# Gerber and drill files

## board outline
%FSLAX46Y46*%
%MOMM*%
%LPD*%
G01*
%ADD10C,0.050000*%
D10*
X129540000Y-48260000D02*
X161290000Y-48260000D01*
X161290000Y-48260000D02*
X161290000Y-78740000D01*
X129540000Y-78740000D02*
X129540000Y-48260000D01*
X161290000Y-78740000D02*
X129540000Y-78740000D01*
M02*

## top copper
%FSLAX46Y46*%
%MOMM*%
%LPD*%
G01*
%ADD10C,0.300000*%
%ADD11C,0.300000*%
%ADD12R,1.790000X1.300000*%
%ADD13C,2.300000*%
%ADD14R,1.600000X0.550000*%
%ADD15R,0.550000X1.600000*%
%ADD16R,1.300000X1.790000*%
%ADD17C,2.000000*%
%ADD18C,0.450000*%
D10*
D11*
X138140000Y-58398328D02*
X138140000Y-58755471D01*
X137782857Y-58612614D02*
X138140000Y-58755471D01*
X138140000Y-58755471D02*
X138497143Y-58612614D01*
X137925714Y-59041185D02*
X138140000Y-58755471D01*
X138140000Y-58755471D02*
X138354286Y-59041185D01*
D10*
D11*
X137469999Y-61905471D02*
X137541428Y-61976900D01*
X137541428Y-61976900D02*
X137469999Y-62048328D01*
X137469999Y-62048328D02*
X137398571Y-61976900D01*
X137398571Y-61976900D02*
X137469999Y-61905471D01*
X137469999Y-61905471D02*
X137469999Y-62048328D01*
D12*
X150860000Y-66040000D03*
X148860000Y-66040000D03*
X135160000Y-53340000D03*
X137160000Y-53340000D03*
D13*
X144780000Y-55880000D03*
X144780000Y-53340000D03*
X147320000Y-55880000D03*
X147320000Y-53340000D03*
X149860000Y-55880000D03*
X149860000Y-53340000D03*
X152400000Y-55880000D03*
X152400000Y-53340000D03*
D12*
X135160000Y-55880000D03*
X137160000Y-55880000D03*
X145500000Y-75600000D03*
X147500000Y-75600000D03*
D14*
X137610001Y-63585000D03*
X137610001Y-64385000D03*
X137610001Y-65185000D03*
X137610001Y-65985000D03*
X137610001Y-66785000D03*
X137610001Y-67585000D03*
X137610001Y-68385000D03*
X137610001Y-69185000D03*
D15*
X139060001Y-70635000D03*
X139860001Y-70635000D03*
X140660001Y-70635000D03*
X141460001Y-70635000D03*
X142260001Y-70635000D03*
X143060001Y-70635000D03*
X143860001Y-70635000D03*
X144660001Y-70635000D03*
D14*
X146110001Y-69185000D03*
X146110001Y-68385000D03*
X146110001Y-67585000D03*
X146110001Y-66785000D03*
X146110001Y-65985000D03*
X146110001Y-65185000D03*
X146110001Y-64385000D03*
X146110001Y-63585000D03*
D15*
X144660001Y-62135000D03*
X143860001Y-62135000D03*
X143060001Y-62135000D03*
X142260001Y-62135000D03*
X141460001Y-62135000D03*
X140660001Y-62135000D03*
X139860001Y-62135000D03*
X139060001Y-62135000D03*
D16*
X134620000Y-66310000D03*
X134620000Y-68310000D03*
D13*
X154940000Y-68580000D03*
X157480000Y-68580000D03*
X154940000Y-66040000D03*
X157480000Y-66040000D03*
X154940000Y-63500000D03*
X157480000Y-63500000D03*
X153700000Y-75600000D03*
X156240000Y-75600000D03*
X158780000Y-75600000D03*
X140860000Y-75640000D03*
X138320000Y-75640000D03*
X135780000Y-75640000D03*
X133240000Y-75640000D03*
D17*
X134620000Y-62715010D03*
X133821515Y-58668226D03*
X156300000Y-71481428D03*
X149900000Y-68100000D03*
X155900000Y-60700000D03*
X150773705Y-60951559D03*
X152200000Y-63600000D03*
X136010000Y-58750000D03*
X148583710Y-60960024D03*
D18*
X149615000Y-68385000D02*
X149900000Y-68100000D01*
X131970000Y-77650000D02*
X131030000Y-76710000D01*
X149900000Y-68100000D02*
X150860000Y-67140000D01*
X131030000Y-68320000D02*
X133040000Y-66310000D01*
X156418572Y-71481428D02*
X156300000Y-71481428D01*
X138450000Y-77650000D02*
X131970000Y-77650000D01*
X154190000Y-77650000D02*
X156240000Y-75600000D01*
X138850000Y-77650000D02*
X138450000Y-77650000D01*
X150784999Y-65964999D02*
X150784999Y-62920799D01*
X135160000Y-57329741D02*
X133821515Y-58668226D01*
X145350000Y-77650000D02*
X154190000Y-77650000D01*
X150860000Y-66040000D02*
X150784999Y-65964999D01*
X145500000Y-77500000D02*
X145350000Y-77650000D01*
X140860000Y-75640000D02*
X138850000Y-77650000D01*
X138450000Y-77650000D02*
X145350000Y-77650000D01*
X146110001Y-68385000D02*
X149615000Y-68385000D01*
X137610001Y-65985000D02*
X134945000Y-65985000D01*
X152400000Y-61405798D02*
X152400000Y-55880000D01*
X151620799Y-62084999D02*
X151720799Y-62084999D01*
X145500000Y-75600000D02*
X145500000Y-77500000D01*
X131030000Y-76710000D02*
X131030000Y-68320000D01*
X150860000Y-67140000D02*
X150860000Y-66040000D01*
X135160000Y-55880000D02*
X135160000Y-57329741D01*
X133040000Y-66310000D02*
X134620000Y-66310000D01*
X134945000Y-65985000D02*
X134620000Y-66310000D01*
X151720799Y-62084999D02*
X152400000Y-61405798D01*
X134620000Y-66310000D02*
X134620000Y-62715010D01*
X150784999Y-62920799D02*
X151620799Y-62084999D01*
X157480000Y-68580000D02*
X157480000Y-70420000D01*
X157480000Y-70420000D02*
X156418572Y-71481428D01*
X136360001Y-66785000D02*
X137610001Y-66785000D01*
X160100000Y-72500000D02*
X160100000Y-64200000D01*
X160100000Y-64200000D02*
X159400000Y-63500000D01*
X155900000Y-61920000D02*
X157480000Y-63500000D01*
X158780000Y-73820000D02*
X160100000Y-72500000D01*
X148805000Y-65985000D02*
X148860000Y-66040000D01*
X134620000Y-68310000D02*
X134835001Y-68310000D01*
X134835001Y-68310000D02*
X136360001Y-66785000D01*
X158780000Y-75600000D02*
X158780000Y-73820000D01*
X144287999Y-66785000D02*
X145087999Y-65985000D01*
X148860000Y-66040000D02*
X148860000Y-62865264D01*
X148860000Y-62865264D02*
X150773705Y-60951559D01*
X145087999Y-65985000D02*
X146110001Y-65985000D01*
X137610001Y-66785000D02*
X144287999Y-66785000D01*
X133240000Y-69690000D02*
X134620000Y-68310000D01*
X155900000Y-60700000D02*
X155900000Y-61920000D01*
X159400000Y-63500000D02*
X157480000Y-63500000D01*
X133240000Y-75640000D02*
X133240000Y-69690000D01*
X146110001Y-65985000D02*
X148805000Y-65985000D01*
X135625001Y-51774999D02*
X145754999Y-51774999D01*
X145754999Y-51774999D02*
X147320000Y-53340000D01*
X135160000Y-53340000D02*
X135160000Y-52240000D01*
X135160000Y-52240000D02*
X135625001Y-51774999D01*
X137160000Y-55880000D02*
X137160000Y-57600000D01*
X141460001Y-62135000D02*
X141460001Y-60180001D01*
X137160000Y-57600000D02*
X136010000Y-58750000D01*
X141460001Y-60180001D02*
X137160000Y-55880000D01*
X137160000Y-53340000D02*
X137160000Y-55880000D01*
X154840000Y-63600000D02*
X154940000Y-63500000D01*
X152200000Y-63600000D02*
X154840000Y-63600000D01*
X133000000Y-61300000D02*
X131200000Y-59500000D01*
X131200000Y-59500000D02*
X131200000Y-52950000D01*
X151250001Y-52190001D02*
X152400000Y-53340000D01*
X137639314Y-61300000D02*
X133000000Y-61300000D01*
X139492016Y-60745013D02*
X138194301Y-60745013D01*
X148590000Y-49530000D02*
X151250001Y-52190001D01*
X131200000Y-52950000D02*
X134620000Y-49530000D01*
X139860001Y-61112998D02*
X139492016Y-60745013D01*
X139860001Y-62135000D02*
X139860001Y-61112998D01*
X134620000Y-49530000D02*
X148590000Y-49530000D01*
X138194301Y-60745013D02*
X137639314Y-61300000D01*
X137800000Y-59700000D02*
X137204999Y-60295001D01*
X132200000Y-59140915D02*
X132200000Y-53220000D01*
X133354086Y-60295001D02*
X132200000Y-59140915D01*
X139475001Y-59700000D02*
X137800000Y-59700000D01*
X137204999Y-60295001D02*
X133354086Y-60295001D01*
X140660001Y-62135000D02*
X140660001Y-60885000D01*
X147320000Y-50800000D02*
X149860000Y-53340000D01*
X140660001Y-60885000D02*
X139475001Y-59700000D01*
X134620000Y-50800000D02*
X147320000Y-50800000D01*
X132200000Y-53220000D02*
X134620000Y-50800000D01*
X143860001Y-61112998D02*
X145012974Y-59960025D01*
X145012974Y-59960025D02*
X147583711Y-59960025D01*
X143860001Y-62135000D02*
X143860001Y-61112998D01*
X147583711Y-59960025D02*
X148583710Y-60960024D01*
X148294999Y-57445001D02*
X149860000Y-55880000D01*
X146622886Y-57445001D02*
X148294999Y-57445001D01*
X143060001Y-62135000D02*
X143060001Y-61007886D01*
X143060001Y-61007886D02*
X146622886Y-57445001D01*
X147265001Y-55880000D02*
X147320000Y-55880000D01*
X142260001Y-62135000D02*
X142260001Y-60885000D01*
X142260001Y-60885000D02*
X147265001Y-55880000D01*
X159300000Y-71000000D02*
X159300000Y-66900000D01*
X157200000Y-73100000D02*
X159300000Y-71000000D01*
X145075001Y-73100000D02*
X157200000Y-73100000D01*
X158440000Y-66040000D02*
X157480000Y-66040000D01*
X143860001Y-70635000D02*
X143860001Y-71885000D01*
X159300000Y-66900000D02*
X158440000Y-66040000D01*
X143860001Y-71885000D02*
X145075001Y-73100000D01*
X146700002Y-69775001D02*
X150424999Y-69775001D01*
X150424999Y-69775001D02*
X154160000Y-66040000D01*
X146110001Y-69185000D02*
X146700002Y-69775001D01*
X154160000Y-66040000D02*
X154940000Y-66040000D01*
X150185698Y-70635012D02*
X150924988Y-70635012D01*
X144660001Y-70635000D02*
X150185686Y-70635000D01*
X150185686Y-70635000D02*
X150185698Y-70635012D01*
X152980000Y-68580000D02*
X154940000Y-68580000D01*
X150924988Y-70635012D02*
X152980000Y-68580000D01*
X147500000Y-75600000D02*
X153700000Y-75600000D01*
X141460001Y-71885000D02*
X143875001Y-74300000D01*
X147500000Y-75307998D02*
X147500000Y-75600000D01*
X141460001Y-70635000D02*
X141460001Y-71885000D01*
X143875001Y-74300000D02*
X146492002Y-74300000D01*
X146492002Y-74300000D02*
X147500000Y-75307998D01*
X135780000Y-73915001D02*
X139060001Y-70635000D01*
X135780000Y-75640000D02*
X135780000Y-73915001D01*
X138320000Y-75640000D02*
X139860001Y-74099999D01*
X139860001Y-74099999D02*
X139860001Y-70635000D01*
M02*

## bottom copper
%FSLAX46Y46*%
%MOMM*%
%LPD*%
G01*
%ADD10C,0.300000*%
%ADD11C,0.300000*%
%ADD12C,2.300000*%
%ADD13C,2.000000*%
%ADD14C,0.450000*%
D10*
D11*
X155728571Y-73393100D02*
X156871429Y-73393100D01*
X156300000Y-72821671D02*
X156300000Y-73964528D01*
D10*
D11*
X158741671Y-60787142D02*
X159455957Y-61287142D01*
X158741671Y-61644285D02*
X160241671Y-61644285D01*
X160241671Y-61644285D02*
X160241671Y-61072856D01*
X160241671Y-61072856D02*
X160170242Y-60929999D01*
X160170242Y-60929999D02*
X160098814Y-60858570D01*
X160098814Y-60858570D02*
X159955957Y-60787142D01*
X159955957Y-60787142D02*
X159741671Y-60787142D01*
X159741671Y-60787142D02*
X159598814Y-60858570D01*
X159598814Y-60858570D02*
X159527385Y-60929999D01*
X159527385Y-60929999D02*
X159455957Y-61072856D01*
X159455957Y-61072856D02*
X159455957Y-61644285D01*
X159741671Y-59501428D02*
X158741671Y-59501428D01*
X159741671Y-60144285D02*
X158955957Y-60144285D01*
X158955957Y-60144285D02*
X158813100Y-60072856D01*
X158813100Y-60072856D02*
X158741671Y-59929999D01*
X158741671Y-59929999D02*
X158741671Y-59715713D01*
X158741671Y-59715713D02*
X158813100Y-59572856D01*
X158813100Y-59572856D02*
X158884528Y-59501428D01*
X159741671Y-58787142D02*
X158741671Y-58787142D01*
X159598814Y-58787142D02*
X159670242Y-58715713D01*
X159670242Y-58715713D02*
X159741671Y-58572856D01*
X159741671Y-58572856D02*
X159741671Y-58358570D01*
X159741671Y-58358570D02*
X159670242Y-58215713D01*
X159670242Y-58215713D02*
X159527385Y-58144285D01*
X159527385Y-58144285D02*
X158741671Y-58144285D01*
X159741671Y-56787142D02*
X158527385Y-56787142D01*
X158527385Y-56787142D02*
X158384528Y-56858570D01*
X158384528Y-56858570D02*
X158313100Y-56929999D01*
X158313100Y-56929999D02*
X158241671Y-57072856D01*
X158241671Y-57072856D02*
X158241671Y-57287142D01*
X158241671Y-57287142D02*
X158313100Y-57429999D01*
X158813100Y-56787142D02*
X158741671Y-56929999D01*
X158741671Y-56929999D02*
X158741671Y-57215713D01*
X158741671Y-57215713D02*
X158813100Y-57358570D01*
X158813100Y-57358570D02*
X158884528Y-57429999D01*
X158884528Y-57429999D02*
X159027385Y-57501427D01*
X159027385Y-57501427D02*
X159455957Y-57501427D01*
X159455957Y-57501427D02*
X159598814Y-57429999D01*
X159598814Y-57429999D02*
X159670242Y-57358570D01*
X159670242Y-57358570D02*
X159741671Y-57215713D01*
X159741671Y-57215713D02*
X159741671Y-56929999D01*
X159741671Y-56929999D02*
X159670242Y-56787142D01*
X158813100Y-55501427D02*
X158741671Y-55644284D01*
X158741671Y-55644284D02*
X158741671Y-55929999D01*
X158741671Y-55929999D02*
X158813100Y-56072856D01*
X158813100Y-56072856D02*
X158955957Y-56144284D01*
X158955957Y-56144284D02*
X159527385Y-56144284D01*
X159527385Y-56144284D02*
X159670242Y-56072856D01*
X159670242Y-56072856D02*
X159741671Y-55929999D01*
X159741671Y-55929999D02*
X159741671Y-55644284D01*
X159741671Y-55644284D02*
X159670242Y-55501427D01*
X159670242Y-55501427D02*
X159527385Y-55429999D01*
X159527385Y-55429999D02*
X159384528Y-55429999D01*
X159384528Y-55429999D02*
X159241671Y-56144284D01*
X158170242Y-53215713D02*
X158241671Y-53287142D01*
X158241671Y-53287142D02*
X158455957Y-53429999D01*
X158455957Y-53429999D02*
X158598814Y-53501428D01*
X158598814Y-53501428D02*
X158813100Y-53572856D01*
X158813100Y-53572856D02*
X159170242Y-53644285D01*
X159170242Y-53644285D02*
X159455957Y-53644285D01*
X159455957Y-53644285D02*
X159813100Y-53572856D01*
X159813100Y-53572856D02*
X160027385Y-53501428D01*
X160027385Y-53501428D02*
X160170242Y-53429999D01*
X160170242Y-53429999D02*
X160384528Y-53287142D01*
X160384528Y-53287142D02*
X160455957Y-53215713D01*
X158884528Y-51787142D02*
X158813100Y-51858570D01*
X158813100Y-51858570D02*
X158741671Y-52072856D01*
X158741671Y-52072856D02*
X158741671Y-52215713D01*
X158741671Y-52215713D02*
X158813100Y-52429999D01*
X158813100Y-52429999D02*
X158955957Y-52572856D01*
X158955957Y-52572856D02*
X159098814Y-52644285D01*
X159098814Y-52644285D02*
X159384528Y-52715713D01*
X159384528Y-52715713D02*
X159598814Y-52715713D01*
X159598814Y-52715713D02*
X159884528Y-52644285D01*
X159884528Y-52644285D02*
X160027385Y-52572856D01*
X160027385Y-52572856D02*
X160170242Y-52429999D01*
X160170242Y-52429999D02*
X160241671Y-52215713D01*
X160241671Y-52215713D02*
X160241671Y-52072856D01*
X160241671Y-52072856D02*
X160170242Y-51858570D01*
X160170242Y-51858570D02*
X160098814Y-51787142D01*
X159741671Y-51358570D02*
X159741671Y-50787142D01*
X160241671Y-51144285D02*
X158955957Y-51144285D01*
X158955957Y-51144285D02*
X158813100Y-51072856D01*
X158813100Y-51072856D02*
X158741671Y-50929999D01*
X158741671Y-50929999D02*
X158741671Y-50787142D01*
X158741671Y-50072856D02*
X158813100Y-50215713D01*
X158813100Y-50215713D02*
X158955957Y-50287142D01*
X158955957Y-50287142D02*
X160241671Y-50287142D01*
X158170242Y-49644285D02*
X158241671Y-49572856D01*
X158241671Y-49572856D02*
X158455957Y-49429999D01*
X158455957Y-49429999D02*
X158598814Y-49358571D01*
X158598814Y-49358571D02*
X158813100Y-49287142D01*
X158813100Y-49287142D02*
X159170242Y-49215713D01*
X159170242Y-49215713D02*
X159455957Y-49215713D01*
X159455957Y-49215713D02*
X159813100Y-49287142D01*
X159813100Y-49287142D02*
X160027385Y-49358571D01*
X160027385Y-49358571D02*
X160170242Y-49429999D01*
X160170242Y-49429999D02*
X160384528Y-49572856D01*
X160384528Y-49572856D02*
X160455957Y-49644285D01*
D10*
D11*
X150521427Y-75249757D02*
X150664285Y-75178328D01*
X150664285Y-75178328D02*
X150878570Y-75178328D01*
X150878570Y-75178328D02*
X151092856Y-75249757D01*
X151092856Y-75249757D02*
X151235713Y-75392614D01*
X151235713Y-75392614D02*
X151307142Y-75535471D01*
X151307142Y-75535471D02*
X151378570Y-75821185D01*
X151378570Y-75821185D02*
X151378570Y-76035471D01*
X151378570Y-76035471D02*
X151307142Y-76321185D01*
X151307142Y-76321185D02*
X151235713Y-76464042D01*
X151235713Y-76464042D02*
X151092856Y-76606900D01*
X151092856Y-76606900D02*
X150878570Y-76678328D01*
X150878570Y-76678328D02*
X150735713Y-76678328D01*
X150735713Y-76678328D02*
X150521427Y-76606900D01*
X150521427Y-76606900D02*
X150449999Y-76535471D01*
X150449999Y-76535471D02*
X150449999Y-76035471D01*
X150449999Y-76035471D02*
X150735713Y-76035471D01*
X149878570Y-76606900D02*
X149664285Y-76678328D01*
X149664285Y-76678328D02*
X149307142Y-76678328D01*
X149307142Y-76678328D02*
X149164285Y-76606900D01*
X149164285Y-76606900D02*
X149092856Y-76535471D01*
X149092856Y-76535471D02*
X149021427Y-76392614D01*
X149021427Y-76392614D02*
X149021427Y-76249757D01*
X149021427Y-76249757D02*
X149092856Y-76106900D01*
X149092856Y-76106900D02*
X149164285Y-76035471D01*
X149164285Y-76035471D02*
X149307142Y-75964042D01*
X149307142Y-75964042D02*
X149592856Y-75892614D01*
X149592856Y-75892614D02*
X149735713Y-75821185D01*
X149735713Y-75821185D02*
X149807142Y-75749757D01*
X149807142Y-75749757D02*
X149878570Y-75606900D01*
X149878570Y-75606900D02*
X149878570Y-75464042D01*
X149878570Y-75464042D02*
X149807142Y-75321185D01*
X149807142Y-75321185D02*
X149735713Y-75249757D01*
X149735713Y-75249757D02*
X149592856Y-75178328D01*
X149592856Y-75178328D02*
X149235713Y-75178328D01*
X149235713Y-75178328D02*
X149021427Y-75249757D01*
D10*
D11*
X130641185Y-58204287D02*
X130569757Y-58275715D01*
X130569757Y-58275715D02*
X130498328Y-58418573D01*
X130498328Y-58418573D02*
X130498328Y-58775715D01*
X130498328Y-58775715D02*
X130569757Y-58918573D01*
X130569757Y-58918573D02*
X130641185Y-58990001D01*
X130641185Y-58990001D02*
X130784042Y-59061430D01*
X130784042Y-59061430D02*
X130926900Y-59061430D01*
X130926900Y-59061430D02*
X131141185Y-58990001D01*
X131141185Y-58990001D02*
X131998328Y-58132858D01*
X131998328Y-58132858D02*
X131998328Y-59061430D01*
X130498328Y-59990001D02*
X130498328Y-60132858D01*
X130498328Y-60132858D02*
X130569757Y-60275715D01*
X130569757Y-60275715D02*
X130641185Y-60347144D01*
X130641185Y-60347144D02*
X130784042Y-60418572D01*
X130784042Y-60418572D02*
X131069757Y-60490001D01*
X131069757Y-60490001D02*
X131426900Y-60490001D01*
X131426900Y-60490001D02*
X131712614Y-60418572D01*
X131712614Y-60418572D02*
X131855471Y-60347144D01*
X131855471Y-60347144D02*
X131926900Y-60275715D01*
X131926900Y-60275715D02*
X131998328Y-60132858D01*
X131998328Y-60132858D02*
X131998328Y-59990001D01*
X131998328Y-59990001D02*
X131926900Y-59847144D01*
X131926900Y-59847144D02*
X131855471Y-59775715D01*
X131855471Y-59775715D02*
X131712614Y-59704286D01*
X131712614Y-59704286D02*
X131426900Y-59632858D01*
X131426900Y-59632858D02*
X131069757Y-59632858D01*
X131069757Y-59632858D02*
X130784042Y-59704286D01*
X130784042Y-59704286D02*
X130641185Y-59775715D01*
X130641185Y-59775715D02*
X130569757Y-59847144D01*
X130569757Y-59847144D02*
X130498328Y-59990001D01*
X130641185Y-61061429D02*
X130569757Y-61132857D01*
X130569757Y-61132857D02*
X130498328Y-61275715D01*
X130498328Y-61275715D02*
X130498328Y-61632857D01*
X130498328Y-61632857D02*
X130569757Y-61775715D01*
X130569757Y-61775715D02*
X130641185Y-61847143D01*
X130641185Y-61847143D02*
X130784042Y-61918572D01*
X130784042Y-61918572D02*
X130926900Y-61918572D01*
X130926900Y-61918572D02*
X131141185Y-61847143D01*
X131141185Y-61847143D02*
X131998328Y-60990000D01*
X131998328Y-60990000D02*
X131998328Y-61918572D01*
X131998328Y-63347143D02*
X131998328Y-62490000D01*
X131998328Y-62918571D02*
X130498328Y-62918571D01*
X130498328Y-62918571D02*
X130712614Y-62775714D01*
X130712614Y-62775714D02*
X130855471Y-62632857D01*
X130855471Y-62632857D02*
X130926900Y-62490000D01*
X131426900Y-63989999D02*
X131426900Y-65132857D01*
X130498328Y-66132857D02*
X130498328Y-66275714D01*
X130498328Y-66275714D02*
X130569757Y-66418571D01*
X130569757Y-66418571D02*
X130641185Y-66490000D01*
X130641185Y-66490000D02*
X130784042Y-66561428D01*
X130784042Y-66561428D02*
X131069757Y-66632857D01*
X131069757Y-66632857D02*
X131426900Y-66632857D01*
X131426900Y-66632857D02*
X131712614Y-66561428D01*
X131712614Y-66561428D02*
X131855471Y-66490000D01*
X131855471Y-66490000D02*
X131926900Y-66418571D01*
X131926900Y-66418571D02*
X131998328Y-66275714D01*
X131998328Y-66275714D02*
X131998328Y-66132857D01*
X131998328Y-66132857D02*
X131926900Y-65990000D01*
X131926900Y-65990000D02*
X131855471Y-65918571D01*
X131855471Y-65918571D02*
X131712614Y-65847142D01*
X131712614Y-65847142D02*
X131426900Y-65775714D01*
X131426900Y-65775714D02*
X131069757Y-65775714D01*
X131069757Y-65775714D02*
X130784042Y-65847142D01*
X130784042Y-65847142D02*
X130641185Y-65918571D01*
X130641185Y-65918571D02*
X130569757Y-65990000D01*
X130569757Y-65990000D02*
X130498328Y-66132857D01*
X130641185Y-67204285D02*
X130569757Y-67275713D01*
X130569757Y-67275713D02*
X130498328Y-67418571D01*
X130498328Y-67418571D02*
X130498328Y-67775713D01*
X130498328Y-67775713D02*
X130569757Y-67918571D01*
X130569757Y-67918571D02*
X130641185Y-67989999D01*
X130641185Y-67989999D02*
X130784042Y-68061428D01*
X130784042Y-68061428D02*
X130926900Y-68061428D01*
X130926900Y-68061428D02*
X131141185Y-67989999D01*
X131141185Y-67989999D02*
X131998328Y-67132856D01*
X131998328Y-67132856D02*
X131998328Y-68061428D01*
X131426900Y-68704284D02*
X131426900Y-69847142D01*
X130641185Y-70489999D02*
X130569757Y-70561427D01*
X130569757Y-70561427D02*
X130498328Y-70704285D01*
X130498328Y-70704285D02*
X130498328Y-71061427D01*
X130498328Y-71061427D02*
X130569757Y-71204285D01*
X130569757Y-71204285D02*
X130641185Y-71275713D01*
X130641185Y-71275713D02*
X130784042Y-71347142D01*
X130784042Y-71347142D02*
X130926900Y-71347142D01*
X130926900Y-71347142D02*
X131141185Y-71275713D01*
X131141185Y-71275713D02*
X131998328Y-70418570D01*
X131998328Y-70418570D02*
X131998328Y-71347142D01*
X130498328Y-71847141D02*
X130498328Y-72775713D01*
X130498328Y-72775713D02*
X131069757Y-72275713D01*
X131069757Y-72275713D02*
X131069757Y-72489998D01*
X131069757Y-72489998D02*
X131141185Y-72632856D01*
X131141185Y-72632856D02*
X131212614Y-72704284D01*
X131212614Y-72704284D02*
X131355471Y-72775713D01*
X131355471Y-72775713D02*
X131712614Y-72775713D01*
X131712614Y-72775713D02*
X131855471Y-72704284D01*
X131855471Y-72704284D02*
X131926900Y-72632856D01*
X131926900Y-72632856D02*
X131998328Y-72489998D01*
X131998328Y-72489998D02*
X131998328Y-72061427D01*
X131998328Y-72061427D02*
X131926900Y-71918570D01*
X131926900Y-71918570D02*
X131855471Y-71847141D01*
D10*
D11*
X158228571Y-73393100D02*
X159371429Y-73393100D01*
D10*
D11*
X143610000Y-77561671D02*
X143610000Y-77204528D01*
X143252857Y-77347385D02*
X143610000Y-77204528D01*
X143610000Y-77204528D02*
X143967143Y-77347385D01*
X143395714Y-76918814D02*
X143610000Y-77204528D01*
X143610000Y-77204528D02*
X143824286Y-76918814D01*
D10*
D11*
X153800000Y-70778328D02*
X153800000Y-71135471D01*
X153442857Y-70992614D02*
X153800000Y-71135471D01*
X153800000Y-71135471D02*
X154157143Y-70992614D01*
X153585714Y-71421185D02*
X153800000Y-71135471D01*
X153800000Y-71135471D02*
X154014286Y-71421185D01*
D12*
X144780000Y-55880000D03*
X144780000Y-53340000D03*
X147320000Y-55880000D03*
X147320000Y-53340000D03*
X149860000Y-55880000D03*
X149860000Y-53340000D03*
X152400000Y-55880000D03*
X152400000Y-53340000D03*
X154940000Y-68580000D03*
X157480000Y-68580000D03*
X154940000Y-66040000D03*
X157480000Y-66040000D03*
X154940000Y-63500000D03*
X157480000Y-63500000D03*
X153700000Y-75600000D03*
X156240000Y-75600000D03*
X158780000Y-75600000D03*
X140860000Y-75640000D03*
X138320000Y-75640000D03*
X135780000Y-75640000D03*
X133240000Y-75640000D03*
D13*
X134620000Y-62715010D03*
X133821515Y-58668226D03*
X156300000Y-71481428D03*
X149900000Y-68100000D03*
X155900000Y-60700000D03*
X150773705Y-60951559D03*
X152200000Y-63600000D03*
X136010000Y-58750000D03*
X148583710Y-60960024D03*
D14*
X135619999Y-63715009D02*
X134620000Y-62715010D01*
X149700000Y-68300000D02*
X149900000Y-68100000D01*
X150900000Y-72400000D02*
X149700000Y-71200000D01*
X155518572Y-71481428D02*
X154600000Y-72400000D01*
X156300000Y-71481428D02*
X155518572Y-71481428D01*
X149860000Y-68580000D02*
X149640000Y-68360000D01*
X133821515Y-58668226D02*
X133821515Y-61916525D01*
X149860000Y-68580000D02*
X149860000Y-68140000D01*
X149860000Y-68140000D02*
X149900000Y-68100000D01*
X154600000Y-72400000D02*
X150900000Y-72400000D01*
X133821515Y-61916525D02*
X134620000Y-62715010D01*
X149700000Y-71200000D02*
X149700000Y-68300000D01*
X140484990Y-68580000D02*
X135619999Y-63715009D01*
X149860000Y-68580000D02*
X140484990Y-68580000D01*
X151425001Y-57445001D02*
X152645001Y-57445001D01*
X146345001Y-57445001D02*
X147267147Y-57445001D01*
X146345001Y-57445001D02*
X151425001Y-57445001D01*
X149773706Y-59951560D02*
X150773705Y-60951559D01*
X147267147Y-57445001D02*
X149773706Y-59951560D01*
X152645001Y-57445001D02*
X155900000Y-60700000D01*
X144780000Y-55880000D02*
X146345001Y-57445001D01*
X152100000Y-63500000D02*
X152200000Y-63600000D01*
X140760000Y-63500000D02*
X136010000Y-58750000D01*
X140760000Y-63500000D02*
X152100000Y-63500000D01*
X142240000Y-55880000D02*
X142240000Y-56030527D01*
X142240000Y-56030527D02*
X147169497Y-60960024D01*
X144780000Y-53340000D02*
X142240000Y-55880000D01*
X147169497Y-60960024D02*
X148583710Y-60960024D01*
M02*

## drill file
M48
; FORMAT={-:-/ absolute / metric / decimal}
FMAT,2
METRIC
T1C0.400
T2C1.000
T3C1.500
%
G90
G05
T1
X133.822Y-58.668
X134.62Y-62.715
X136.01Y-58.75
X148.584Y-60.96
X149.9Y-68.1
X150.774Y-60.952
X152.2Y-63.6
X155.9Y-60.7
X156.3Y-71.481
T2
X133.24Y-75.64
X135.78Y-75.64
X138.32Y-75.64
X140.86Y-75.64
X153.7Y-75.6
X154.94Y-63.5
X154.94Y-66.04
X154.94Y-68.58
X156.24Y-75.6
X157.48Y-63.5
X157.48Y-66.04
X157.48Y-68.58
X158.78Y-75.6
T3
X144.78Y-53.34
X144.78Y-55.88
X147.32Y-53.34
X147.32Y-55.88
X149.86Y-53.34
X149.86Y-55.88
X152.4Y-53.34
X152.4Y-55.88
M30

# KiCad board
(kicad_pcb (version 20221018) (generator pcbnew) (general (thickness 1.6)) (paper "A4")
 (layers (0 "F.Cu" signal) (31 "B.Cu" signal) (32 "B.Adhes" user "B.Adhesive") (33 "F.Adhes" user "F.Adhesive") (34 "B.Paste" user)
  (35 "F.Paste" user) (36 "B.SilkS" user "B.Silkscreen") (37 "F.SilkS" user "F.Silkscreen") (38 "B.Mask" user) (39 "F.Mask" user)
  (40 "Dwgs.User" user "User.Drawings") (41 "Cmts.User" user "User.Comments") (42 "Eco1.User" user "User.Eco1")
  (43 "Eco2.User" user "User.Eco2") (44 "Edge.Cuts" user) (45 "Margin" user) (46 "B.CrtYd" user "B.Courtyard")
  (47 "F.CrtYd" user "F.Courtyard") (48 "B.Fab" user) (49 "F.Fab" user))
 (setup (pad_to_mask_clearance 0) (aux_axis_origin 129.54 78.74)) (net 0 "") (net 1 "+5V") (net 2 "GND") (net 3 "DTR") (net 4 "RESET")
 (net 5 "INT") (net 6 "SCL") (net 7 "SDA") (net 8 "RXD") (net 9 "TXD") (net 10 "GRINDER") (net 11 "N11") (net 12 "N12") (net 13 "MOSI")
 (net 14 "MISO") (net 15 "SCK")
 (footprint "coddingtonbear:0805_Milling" (layer "F.Cu") (at 149.86 66.04 180)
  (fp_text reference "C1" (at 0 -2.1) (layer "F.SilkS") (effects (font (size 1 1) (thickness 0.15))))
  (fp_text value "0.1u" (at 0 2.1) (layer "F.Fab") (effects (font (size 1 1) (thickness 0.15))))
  (pad "1" smd rect (at -1 0 180) (size 1.79 1.3) (layers "F.Cu" "F.Paste" "F.Mask") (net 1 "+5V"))
  (pad "2" smd rect (at 1 0 180) (size 1.79 1.3) (layers "F.Cu" "F.Paste" "F.Mask") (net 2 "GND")))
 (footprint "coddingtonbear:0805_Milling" (layer "F.Cu") (at 136.16 53.34)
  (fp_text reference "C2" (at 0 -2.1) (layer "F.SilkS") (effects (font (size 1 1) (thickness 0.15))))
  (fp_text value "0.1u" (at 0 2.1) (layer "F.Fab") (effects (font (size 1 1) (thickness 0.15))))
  (pad "1" smd rect (at -1 0) (size 1.79 1.3) (layers "F.Cu" "F.Paste" "F.Mask") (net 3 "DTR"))
  (pad "2" smd rect (at 1 0) (size 1.79 1.3) (layers "F.Cu" "F.Paste" "F.Mask") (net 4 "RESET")))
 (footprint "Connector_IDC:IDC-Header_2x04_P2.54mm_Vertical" (layer "F.Cu") (at 144.78 55.88 90)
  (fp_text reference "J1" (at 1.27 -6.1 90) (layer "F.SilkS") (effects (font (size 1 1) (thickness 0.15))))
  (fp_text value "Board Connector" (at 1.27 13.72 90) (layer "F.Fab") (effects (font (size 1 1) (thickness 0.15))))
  (pad "1" thru_hole circle (at 0 0 90) (size 2.3 2.3) (drill 1.5) (layers "*.Cu" "*.Mask") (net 2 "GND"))
  (pad "2" thru_hole circle (at 2.54 0 90) (size 2.3 2.3) (drill 1.5) (layers "*.Cu" "*.Mask") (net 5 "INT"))
  (pad "3" thru_hole circle (at 0 2.54 90) (size 2.3 2.3) (drill 1.5) (layers "*.Cu" "*.Mask") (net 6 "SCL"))
  (pad "4" thru_hole circle (at 2.54 2.54 90) (size 2.3 2.3) (drill 1.5) (layers "*.Cu" "*.Mask") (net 3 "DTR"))
  (pad "5" thru_hole circle (at 0 5.08 90) (size 2.3 2.3) (drill 1.5) (layers "*.Cu" "*.Mask") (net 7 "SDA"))
  (pad "6" thru_hole circle (at 2.54 5.08 90) (size 2.3 2.3) (drill 1.5) (layers "*.Cu" "*.Mask") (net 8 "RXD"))
  (pad "7" thru_hole circle (at 0 7.62 90) (size 2.3 2.3) (drill 1.5) (layers "*.Cu" "*.Mask") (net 1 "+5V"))
  (pad "8" thru_hole circle (at 2.54 7.62 90) (size 2.3 2.3) (drill 1.5) (layers "*.Cu" "*.Mask") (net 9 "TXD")))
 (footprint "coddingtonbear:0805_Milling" (layer "F.Cu") (at 136.16 55.88)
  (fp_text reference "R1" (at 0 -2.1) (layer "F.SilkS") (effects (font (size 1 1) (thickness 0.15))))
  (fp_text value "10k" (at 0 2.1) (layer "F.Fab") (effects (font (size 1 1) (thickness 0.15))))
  (pad "1" smd rect (at -1 0) (size 1.79 1.3) (layers "F.Cu" "F.Paste" "F.Mask") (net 1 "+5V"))
  (pad "2" smd rect (at 1 0) (size 1.79 1.3) (layers "F.Cu" "F.Paste" "F.Mask") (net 4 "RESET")))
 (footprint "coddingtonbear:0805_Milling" (layer "F.Cu") (at 146.5 75.6)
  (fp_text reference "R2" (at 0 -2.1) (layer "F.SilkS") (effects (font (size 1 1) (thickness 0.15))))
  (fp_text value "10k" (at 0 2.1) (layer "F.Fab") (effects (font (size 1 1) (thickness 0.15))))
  (pad "1" smd rect (at -1 0) (size 1.79 1.3) (layers "F.Cu" "F.Paste" "F.Mask") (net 1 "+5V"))
  (pad "2" smd rect (at 1 0) (size 1.79 1.3) (layers "F.Cu" "F.Paste" "F.Mask") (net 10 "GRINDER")))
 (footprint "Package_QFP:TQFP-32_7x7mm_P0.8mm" (layer "F.Cu") (at 141.860001 66.385)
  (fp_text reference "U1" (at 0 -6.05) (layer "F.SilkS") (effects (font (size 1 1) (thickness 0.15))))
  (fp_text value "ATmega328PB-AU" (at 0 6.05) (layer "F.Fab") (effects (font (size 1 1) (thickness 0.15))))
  (pad "1" smd rect (at -4.25 -2.8) (size 1.6 0.55) (layers "F.Cu" "F.Paste" "F.Mask"))
  (pad "2" smd rect (at -4.25 -2) (size 1.6 0.55) (layers "F.Cu" "F.Paste" "F.Mask"))
  (pad "3" smd rect (at -4.25 -1.2) (size 1.6 0.55) (layers "F.Cu" "F.Paste" "F.Mask"))
  (pad "4" smd rect (at -4.25 -0.4) (size 1.6 0.55) (layers "F.Cu" "F.Paste" "F.Mask") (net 1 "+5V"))
  (pad "5" smd rect (at -4.25 0.4) (size 1.6 0.55) (layers "F.Cu" "F.Paste" "F.Mask") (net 2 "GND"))
  (pad "6" smd rect (at -4.25 1.2) (size 1.6 0.55) (layers "F.Cu" "F.Paste" "F.Mask"))
  (pad "7" smd rect (at -4.25 2) (size 1.6 0.55) (layers "F.Cu" "F.Paste" "F.Mask"))
  (pad "8" smd rect (at -4.25 2.8) (size 1.6 0.55) (layers "F.Cu" "F.Paste" "F.Mask"))
  (pad "9" smd rect (at -2.8 4.25 90) (size 1.6 0.55) (layers "F.Cu" "F.Paste" "F.Mask") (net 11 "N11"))
  (pad "10" smd rect (at -2 4.25 90) (size 1.6 0.55) (layers "F.Cu" "F.Paste" "F.Mask") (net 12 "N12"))
  (pad "11" smd rect (at -1.2 4.25 90) (size 1.6 0.55) (layers "F.Cu" "F.Paste" "F.Mask"))
  (pad "12" smd rect (at -0.4 4.25 90) (size 1.6 0.55) (layers "F.Cu" "F.Paste" "F.Mask") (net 10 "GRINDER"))
  (pad "13" smd rect (at 0.4 4.25 90) (size 1.6 0.55) (layers "F.Cu" "F.Paste" "F.Mask"))
  (pad "14" smd rect (at 1.2 4.25 90) (size 1.6 0.55) (layers "F.Cu" "F.Paste" "F.Mask"))
  (pad "15" smd rect (at 2 4.25 90) (size 1.6 0.55) (layers "F.Cu" "F.Paste" "F.Mask") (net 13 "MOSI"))
  (pad "16" smd rect (at 2.8 4.25 90) (size 1.6 0.55) (layers "F.Cu" "F.Paste" "F.Mask") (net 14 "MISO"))
  (pad "17" smd rect (at 4.25 2.8) (size 1.6 0.55) (layers "F.Cu" "F.Paste" "F.Mask") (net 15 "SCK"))
  (pad "18" smd rect (at 4.25 2) (size 1.6 0.55) (layers "F.Cu" "F.Paste" "F.Mask") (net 1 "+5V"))
  (pad "19" smd rect (at 4.25 1.2) (size 1.6 0.55) (layers "F.Cu" "F.Paste" "F.Mask"))
  (pad "20" smd rect (at 4.25 0.4) (size 1.6 0.55) (layers "F.Cu" "F.Paste" "F.Mask"))
  (pad "21" smd rect (at 4.25 -0.4) (size 1.6 0.55) (layers "F.Cu" "F.Paste" "F.Mask") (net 2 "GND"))
  (pad "22" smd rect (at 4.25 -1.2) (size 1.6 0.55) (layers "F.Cu" "F.Paste" "F.Mask"))
  (pad "23" smd rect (at 4.25 -2) (size 1.6 0.55) (layers "F.Cu" "F.Paste" "F.Mask"))
  (pad "24" smd rect (at 4.25 -2.8) (size 1.6 0.55) (layers "F.Cu" "F.Paste" "F.Mask"))
  (pad "25" smd rect (at 2.8 -4.25 90) (size 1.6 0.55) (layers "F.Cu" "F.Paste" "F.Mask"))
  (pad "26" smd rect (at 2 -4.25 90) (size 1.6 0.55) (layers "F.Cu" "F.Paste" "F.Mask") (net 5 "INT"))
  (pad "27" smd rect (at 1.2 -4.25 90) (size 1.6 0.55) (layers "F.Cu" "F.Paste" "F.Mask") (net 7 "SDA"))
  (pad "28" smd rect (at 0.4 -4.25 90) (size 1.6 0.55) (layers "F.Cu" "F.Paste" "F.Mask") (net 6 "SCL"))
  (pad "29" smd rect (at -0.4 -4.25 90) (size 1.6 0.55) (layers "F.Cu" "F.Paste" "F.Mask") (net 4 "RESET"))
  (pad "30" smd rect (at -1.2 -4.25 90) (size 1.6 0.55) (layers "F.Cu" "F.Paste" "F.Mask") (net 8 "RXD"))
  (pad "31" smd rect (at -2 -4.25 90) (size 1.6 0.55) (layers "F.Cu" "F.Paste" "F.Mask") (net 9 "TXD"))
  (pad "32" smd rect (at -2.8 -4.25 90) (size 1.6 0.55) (layers "F.Cu" "F.Paste" "F.Mask")))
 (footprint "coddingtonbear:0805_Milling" (layer "F.Cu") (at 134.62 67.31 -90)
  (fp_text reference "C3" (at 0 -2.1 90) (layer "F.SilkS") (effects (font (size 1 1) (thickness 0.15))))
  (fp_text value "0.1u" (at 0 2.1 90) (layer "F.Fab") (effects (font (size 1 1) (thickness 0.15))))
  (pad "1" smd rect (at -1 0 270) (size 1.79 1.3) (layers "F.Cu" "F.Paste" "F.Mask") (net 1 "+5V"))
  (pad "2" smd rect (at 1 0 270) (size 1.79 1.3) (layers "F.Cu" "F.Paste" "F.Mask") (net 2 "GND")))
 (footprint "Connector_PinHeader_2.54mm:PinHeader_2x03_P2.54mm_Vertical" (layer "B.Cu") (at 154.94 68.58)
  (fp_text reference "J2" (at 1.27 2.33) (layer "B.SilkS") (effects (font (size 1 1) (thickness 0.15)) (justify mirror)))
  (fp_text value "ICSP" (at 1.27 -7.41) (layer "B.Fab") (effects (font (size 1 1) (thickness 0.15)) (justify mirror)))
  (pad "1" thru_hole circle (at 0 0) (size 2.3 2.3) (drill 1) (layers "*.Cu" "*.Mask") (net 14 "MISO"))
  (pad "2" thru_hole circle (at 2.54 0) (size 2.3 2.3) (drill 1) (layers "*.Cu" "*.Mask") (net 1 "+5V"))
  (pad "3" thru_hole circle (at 0 -2.54) (size 2.3 2.3) (drill 1) (layers "*.Cu" "*.Mask") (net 15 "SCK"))
  (pad "4" thru_hole circle (at 2.54 -2.54) (size 2.3 2.3) (drill 1) (layers "*.Cu" "*.Mask") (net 13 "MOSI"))
  (pad "5" thru_hole circle (at 0 -5.08) (size 2.3 2.3) (drill 1) (layers "*.Cu" "*.Mask") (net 4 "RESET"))
  (pad "6" thru_hole circle (at 2.54 -5.08) (size 2.3 2.3) (drill 1) (layers "*.Cu" "*.Mask") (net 2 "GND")))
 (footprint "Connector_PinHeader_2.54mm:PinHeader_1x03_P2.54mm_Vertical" (layer "B.Cu") (at 153.7 75.6 -90)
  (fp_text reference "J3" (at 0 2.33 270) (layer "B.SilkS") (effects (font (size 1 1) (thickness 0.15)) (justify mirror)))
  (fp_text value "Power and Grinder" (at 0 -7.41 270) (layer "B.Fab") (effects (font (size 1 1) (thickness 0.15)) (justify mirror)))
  (pad "1" thru_hole circle (at 0 0 270) (size 2.3 2.3) (drill 1) (layers "*.Cu" "*.Mask") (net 10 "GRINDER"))
  (pad "2" thru_hole circle (at 0 -2.54 270) (size 2.3 2.3) (drill 1) (layers "*.Cu" "*.Mask") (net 1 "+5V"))
  (pad "3" thru_hole circle (at 0 -5.08 270) (size 2.3 2.3) (drill 1) (layers "*.Cu" "*.Mask") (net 2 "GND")))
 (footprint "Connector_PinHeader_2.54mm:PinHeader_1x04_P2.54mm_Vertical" (layer "B.Cu") (at 140.86 75.64 90)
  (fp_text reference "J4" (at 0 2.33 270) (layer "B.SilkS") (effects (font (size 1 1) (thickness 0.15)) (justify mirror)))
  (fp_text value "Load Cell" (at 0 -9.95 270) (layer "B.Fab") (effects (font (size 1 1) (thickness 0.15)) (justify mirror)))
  (pad "1" thru_hole circle (at 0 0 90) (size 2.3 2.3) (drill 1) (layers "*.Cu" "*.Mask") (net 1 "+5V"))
  (pad "2" thru_hole circle (at 0 -2.54 90) (size 2.3 2.3) (drill 1) (layers "*.Cu" "*.Mask") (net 12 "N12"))
  (pad "3" thru_hole circle (at 0 -5.08 90) (size 2.3 2.3) (drill 1) (layers "*.Cu" "*.Mask") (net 11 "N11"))
  (pad "4" thru_hole circle (at 0 -7.62 90) (size 2.3 2.3) (drill 1) (layers "*.Cu" "*.Mask") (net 2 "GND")))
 (gr_line (start 129.54 48.26) (end 161.29 48.26) (stroke (width 0.05) (type solid)) (layer "Edge.Cuts"))
 (gr_line (start 161.29 48.26) (end 161.29 78.74) (stroke (width 0.05) (type solid)) (layer "Edge.Cuts"))
 (gr_line (start 129.54 78.74) (end 129.54 48.26) (stroke (width 0.05) (type solid)) (layer "Edge.Cuts"))
 (gr_line (start 161.29 78.74) (end 129.54 78.74) (stroke (width 0.05) (type solid)) (layer "Edge.Cuts"))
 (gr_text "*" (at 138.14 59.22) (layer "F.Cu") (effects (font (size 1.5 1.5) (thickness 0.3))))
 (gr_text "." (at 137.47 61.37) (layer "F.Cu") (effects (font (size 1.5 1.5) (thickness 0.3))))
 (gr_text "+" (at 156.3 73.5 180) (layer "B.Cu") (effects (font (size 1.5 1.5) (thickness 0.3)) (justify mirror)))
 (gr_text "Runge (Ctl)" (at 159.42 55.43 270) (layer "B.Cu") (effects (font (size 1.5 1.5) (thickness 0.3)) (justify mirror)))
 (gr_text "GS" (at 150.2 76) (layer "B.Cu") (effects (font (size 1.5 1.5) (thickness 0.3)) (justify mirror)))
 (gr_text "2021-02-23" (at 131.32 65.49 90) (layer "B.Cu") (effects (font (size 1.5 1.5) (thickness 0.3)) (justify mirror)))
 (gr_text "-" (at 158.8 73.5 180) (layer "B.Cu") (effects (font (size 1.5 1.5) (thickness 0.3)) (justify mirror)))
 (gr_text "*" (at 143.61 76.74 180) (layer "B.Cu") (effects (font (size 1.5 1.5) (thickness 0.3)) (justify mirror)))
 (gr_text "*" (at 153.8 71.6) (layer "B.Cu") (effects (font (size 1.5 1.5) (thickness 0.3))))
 (segment (start 149.615 68.385) (end 149.9 68.1) (width 0.45) (layer "F.Cu") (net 1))
 (segment (start 131.97 77.65) (end 131.03 76.71) (width 0.45) (layer "F.Cu") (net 1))
 (segment (start 149.9 68.1) (end 150.86 67.14) (width 0.45) (layer "F.Cu") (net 1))
 (segment (start 131.03 68.32) (end 133.04 66.31) (width 0.45) (layer "F.Cu") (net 1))
 (segment (start 156.418572 71.481428) (end 156.3 71.481428) (width 0.45) (layer "F.Cu") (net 1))
 (segment (start 138.45 77.65) (end 131.97 77.65) (width 0.45) (layer "F.Cu") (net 1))
 (segment (start 154.19 77.65) (end 156.24 75.6) (width 0.45) (layer "F.Cu") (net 1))
 (segment (start 138.85 77.65) (end 138.45 77.65) (width 0.45) (layer "F.Cu") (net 1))
 (segment (start 150.784999 65.964999) (end 150.784999 62.920799) (width 0.45) (layer "F.Cu") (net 1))
 (segment (start 135.16 57.329741) (end 133.821515 58.668226) (width 0.45) (layer "F.Cu") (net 1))
 (segment (start 145.35 77.65) (end 154.19 77.65) (width 0.45) (layer "F.Cu") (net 1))
 (segment (start 150.86 66.04) (end 150.784999 65.964999) (width 0.45) (layer "F.Cu") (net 1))
 (segment (start 145.5 77.5) (end 145.35 77.65) (width 0.45) (layer "F.Cu") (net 1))
 (segment (start 140.86 75.64) (end 138.85 77.65) (width 0.45) (layer "F.Cu") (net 1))
 (segment (start 138.45 77.65) (end 145.35 77.65) (width 0.45) (layer "F.Cu") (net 1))
 (segment (start 146.110001 68.385) (end 149.615 68.385) (width 0.45) (layer "F.Cu") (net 1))
 (segment (start 137.610001 65.985) (end 134.945 65.985) (width 0.45) (layer "F.Cu") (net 1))
 (segment (start 152.4 61.405798) (end 152.4 55.88) (width 0.45) (layer "F.Cu") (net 1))
 (segment (start 151.620799 62.084999) (end 151.720799 62.084999) (width 0.45) (layer "F.Cu") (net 1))
 (segment (start 145.5 75.6) (end 145.5 77.5) (width 0.45) (layer "F.Cu") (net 1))
 (segment (start 131.03 76.71) (end 131.03 68.32) (width 0.45) (layer "F.Cu") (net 1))
 (segment (start 150.86 67.14) (end 150.86 66.04) (width 0.45) (layer "F.Cu") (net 1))
 (segment (start 135.16 55.88) (end 135.16 57.329741) (width 0.45) (layer "F.Cu") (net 1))
 (segment (start 133.04 66.31) (end 134.62 66.31) (width 0.45) (layer "F.Cu") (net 1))
 (segment (start 134.945 65.985) (end 134.62 66.31) (width 0.45) (layer "F.Cu") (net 1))
 (segment (start 151.720799 62.084999) (end 152.4 61.405798) (width 0.45) (layer "F.Cu") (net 1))
 (segment (start 134.62 66.31) (end 134.62 62.71501) (width 0.45) (layer "F.Cu") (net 1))
 (segment (start 150.784999 62.920799) (end 151.620799 62.084999) (width 0.45) (layer "F.Cu") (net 1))
 (segment (start 157.48 68.58) (end 157.48 70.42) (width 0.45) (layer "F.Cu") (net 1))
 (segment (start 157.48 70.42) (end 156.418572 71.481428) (width 0.45) (layer "F.Cu") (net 1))
 (via (at 134.62 62.71501) (size 2) (drill 0.4) (layers "F.Cu" "B.Cu") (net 1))
 (via (at 133.821515 58.668226) (size 2) (drill 0.4) (layers "F.Cu" "B.Cu") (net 1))
 (via (at 156.3 71.481428) (size 2) (drill 0.4) (layers "F.Cu" "B.Cu") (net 1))
 (via (at 149.9 68.1) (size 2) (drill 0.4) (layers "F.Cu" "B.Cu") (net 1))
 (segment (start 135.619999 63.715009) (end 134.62 62.71501) (width 0.45) (layer "B.Cu") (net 1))
 (segment (start 149.7 68.3) (end 149.9 68.1) (width 0.45) (layer "B.Cu") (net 1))
 (segment (start 150.9 72.4) (end 149.7 71.2) (width 0.45) (layer "B.Cu") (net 1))
 (segment (start 155.518572 71.481428) (end 154.6 72.4) (width 0.45) (layer "B.Cu") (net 1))
 (segment (start 156.3 71.481428) (end 155.518572 71.481428) (width 0.45) (layer "B.Cu") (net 1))
 (segment (start 149.86 68.58) (end 149.64 68.36) (width 0.45) (layer "B.Cu") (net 1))
 (segment (start 133.821515 58.668226) (end 133.821515 61.916525) (width 0.45) (layer "B.Cu") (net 1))
 (segment (start 149.86 68.58) (end 149.86 68.14) (width 0.45) (layer "B.Cu") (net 1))
 (segment (start 149.86 68.14) (end 149.9 68.1) (width 0.45) (layer "B.Cu") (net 1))
 (segment (start 154.6 72.4) (end 150.9 72.4) (width 0.45) (layer "B.Cu") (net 1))
 (segment (start 133.821515 61.916525) (end 134.62 62.71501) (width 0.45) (layer "B.Cu") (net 1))
 (segment (start 149.7 71.2) (end 149.7 68.3) (width 0.45) (layer "B.Cu") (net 1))
 (segment (start 140.48499 68.58) (end 135.619999 63.715009) (width 0.45) (layer "B.Cu") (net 1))
 (segment (start 149.86 68.58) (end 140.48499 68.58) (width 0.45) (layer "B.Cu") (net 1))
 (segment (start 136.360001 66.785) (end 137.610001 66.785) (width 0.45) (layer "F.Cu") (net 2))
 (segment (start 160.1 72.5) (end 160.1 64.2) (width 0.45) (layer "F.Cu") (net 2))
 (segment (start 160.1 64.2) (end 159.4 63.5) (width 0.45) (layer "F.Cu") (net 2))
 (segment (start 155.9 61.92) (end 157.48 63.5) (width 0.45) (layer "F.Cu") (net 2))
 (segment (start 158.78 73.82) (end 160.1 72.5) (width 0.45) (layer "F.Cu") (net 2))
 (segment (start 148.805 65.985) (end 148.86 66.04) (width 0.45) (layer "F.Cu") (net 2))
 (segment (start 134.62 68.31) (end 134.835001 68.31) (width 0.45) (layer "F.Cu") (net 2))
 (segment (start 134.835001 68.31) (end 136.360001 66.785) (width 0.45) (layer "F.Cu") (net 2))
 (segment (start 158.78 75.6) (end 158.78 73.82) (width 0.45) (layer "F.Cu") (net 2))
 (segment (start 144.287999 66.785) (end 145.087999 65.985) (width 0.45) (layer "F.Cu") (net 2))
 (segment (start 148.86 66.04) (end 148.86 62.865264) (width 0.45) (layer "F.Cu") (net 2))
 (segment (start 148.86 62.865264) (end 150.773705 60.951559) (width 0.45) (layer "F.Cu") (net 2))
 (segment (start 145.087999 65.985) (end 146.110001 65.985) (width 0.45) (layer "F.Cu") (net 2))
 (segment (start 137.610001 66.785) (end 144.287999 66.785) (width 0.45) (layer "F.Cu") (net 2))
 (segment (start 133.24 69.69) (end 134.62 68.31) (width 0.45) (layer "F.Cu") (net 2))
 (segment (start 155.9 60.7) (end 155.9 61.92) (width 0.45) (layer "F.Cu") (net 2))
 (segment (start 159.4 63.5) (end 157.48 63.5) (width 0.45) (layer "F.Cu") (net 2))
 (segment (start 133.24 75.64) (end 133.24 69.69) (width 0.45) (layer "F.Cu") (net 2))
 (segment (start 146.110001 65.985) (end 148.805 65.985) (width 0.45) (layer "F.Cu") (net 2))
 (via (at 155.9 60.7) (size 2) (drill 0.4) (layers "F.Cu" "B.Cu") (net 2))
 (via (at 150.773705 60.951559) (size 2) (drill 0.4) (layers "F.Cu" "B.Cu") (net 2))
 (segment (start 151.425001 57.445001) (end 152.645001 57.445001) (width 0.45) (layer "B.Cu") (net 2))
 (segment (start 146.345001 57.445001) (end 147.267147 57.445001) (width 0.45) (layer "B.Cu") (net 2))
 (segment (start 146.345001 57.445001) (end 151.425001 57.445001) (width 0.45) (layer "B.Cu") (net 2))
 (segment (start 149.773706 59.95156) (end 150.773705 60.951559) (width 0.45) (layer "B.Cu") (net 2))
 (segment (start 147.267147 57.445001) (end 149.773706 59.95156) (width 0.45) (layer "B.Cu") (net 2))
 (segment (start 152.645001 57.445001) (end 155.9 60.7) (width 0.45) (layer "B.Cu") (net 2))
 (segment (start 144.78 55.88) (end 146.345001 57.445001) (width 0.45) (layer "B.Cu") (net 2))
 (segment (start 135.625001 51.774999) (end 145.754999 51.774999) (width 0.45) (layer "F.Cu") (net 3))
 (segment (start 145.754999 51.774999) (end 147.32 53.34) (width 0.45) (layer "F.Cu") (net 3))
 (segment (start 135.16 53.34) (end 135.16 52.24) (width 0.45) (layer "F.Cu") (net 3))
 (segment (start 135.16 52.24) (end 135.625001 51.774999) (width 0.45) (layer "F.Cu") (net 3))
 (segment (start 137.16 55.88) (end 137.16 57.6) (width 0.45) (layer "F.Cu") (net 4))
 (segment (start 141.460001 62.135) (end 141.460001 60.180001) (width 0.45) (layer "F.Cu") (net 4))
 (segment (start 137.16 57.6) (end 136.01 58.75) (width 0.45) (layer "F.Cu") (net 4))
 (segment (start 141.460001 60.180001) (end 137.16 55.88) (width 0.45) (layer "F.Cu") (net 4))
 (segment (start 137.16 53.34) (end 137.16 55.88) (width 0.45) (layer "F.Cu") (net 4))
 (segment (start 154.84 63.6) (end 154.94 63.5) (width 0.45) (layer "F.Cu") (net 4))
 (segment (start 152.2 63.6) (end 154.84 63.6) (width 0.45) (layer "F.Cu") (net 4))
 (via (at 152.2 63.6) (size 2) (drill 0.4) (layers "F.Cu" "B.Cu") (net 4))
 (via (at 136.01 58.75) (size 2) (drill 0.4) (layers "F.Cu" "B.Cu") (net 4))
 (segment (start 152.1 63.5) (end 152.2 63.6) (width 0.45) (layer "B.Cu") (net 4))
 (segment (start 140.76 63.5) (end 136.01 58.75) (width 0.45) (layer "B.Cu") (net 4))
 (segment (start 140.76 63.5) (end 152.1 63.5) (width 0.45) (layer "B.Cu") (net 4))
 (segment (start 133 61.3) (end 131.2 59.5) (width 0.45) (layer "F.Cu") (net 9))
 (segment (start 131.2 59.5) (end 131.2 52.95) (width 0.45) (layer "F.Cu") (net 9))
 (segment (start 151.250001 52.190001) (end 152.4 53.34) (width 0.45) (layer "F.Cu") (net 9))
 (segment (start 137.639314 61.3) (end 133 61.3) (width 0.45) (layer "F.Cu") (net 9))
 (segment (start 139.492016 60.745013) (end 138.194301 60.745013) (width 0.45) (layer "F.Cu") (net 9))
 (segment (start 148.59 49.53) (end 151.250001 52.190001) (width 0.45) (layer "F.Cu") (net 9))
 (segment (start 131.2 52.95) (end 134.62 49.53) (width 0.45) (layer "F.Cu") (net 9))
 (segment (start 139.860001 61.112998) (end 139.492016 60.745013) (width 0.45) (layer "F.Cu") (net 9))
 (segment (start 139.860001 62.135) (end 139.860001 61.112998) (width 0.45) (layer "F.Cu") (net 9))
 (segment (start 134.62 49.53) (end 148.59 49.53) (width 0.45) (layer "F.Cu") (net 9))
 (segment (start 138.194301 60.745013) (end 137.639314 61.3) (width 0.45) (layer "F.Cu") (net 9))
 (segment (start 137.8 59.7) (end 137.204999 60.295001) (width 0.45) (layer "F.Cu") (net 8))
 (segment (start 132.2 59.140915) (end 132.2 53.22) (width 0.45) (layer "F.Cu") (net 8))
 (segment (start 133.354086 60.295001) (end 132.2 59.140915) (width 0.45) (layer "F.Cu") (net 8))
 (segment (start 139.475001 59.7) (end 137.8 59.7) (width 0.45) (layer "F.Cu") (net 8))
 (segment (start 137.204999 60.295001) (end 133.354086 60.295001) (width 0.45) (layer "F.Cu") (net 8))
 (segment (start 140.660001 62.135) (end 140.660001 60.885) (width 0.45) (layer "F.Cu") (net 8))
 (segment (start 147.32 50.8) (end 149.86 53.34) (width 0.45) (layer "F.Cu") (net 8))
 (segment (start 140.660001 60.885) (end 139.475001 59.7) (width 0.45) (layer "F.Cu") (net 8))
 (segment (start 134.62 50.8) (end 147.32 50.8) (width 0.45) (layer "F.Cu") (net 8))
 (segment (start 132.2 53.22) (end 134.62 50.8) (width 0.45) (layer "F.Cu") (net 8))
 (segment (start 143.860001 61.112998) (end 145.012974 59.960025) (width 0.45) (layer "F.Cu") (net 5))
 (segment (start 145.012974 59.960025) (end 147.583711 59.960025) (width 0.45) (layer "F.Cu") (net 5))
 (segment (start 143.860001 62.135) (end 143.860001 61.112998) (width 0.45) (layer "F.Cu") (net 5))
 (segment (start 147.583711 59.960025) (end 148.58371 60.960024) (width 0.45) (layer "F.Cu") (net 5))
 (via (at 148.58371 60.960024) (size 2) (drill 0.4) (layers "F.Cu" "B.Cu") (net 5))
 (segment (start 142.24 55.88) (end 142.24 56.030527) (width 0.45) (layer "B.Cu") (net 5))
 (segment (start 142.24 56.030527) (end 147.169497 60.960024) (width 0.45) (layer "B.Cu") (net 5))
 (segment (start 144.78 53.34) (end 142.24 55.88) (width 0.45) (layer "B.Cu") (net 5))
 (segment (start 147.169497 60.960024) (end 148.58371 60.960024) (width 0.45) (layer "B.Cu") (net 5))
 (segment (start 148.294999 57.445001) (end 149.86 55.88) (width 0.45) (layer "F.Cu") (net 7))
 (segment (start 146.622886 57.445001) (end 148.294999 57.445001) (width 0.45) (layer "F.Cu") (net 7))
 (segment (start 143.060001 62.135) (end 143.060001 61.007886) (width 0.45) (layer "F.Cu") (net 7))
 (segment (start 143.060001 61.007886) (end 146.622886 57.445001) (width 0.45) (layer "F.Cu") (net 7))
 (segment (start 147.265001 55.88) (end 147.32 55.88) (width 0.45) (layer "F.Cu") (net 6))
 (segment (start 142.260001 62.135) (end 142.260001 60.885) (width 0.45) (layer "F.Cu") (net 6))
 (segment (start 142.260001 60.885) (end 147.265001 55.88) (width 0.45) (layer "F.Cu") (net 6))
 (segment (start 159.3 71) (end 159.3 66.9) (width 0.45) (layer "F.Cu") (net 13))
 (segment (start 157.2 73.1) (end 159.3 71) (width 0.45) (layer "F.Cu") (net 13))
 (segment (start 145.075001 73.1) (end 157.2 73.1) (width 0.45) (layer "F.Cu") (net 13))
 (segment (start 158.44 66.04) (end 157.48 66.04) (width 0.45) (layer "F.Cu") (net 13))
 (segment (start 143.860001 70.635) (end 143.860001 71.885) (width 0.45) (layer "F.Cu") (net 13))
 (segment (start 159.3 66.9) (end 158.44 66.04) (width 0.45) (layer "F.Cu") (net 13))
 (segment (start 143.860001 71.885) (end 145.075001 73.1) (width 0.45) (layer "F.Cu") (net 13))
 (segment (start 146.700002 69.775001) (end 150.424999 69.775001) (width 0.45) (layer "F.Cu") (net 15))
 (segment (start 150.424999 69.775001) (end 154.16 66.04) (width 0.45) (layer "F.Cu") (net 15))
 (segment (start 146.110001 69.185) (end 146.700002 69.775001) (width 0.45) (layer "F.Cu") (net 15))
 (segment (start 154.16 66.04) (end 154.94 66.04) (width 0.45) (layer "F.Cu") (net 15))
 (segment (start 150.185698 70.635012) (end 150.924988 70.635012) (width 0.45) (layer "F.Cu") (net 14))
 (segment (start 144.660001 70.635) (end 150.185686 70.635) (width 0.45) (layer "F.Cu") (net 14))
 (segment (start 150.185686 70.635) (end 150.185698 70.635012) (width 0.45) (layer "F.Cu") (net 14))
 (segment (start 152.98 68.58) (end 154.94 68.58) (width 0.45) (layer "F.Cu") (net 14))
 (segment (start 150.924988 70.635012) (end 152.98 68.58) (width 0.45) (layer "F.Cu") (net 14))
 (segment (start 147.5 75.6) (end 153.7 75.6) (width 0.45) (layer "F.Cu") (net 10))
 (segment (start 141.460001 71.885) (end 143.875001 74.3) (width 0.45) (layer "F.Cu") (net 10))
 (segment (start 147.5 75.307998) (end 147.5 75.6) (width 0.45) (layer "F.Cu") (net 10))
 (segment (start 141.460001 70.635) (end 141.460001 71.885) (width 0.45) (layer "F.Cu") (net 10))
 (segment (start 143.875001 74.3) (end 146.492002 74.3) (width 0.45) (layer "F.Cu") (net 10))
 (segment (start 146.492002 74.3) (end 147.5 75.307998) (width 0.45) (layer "F.Cu") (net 10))
 (segment (start 135.78 73.915001) (end 139.060001 70.635) (width 0.45) (layer "F.Cu") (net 11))
 (segment (start 135.78 75.64) (end 135.78 73.915001) (width 0.45) (layer "F.Cu") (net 11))
 (segment (start 138.32 75.64) (end 139.860001 74.099999) (width 0.45) (layer "F.Cu") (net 12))
 (segment (start 139.860001 74.099999) (end 139.860001 70.635) (width 0.45) (layer "F.Cu") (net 12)))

